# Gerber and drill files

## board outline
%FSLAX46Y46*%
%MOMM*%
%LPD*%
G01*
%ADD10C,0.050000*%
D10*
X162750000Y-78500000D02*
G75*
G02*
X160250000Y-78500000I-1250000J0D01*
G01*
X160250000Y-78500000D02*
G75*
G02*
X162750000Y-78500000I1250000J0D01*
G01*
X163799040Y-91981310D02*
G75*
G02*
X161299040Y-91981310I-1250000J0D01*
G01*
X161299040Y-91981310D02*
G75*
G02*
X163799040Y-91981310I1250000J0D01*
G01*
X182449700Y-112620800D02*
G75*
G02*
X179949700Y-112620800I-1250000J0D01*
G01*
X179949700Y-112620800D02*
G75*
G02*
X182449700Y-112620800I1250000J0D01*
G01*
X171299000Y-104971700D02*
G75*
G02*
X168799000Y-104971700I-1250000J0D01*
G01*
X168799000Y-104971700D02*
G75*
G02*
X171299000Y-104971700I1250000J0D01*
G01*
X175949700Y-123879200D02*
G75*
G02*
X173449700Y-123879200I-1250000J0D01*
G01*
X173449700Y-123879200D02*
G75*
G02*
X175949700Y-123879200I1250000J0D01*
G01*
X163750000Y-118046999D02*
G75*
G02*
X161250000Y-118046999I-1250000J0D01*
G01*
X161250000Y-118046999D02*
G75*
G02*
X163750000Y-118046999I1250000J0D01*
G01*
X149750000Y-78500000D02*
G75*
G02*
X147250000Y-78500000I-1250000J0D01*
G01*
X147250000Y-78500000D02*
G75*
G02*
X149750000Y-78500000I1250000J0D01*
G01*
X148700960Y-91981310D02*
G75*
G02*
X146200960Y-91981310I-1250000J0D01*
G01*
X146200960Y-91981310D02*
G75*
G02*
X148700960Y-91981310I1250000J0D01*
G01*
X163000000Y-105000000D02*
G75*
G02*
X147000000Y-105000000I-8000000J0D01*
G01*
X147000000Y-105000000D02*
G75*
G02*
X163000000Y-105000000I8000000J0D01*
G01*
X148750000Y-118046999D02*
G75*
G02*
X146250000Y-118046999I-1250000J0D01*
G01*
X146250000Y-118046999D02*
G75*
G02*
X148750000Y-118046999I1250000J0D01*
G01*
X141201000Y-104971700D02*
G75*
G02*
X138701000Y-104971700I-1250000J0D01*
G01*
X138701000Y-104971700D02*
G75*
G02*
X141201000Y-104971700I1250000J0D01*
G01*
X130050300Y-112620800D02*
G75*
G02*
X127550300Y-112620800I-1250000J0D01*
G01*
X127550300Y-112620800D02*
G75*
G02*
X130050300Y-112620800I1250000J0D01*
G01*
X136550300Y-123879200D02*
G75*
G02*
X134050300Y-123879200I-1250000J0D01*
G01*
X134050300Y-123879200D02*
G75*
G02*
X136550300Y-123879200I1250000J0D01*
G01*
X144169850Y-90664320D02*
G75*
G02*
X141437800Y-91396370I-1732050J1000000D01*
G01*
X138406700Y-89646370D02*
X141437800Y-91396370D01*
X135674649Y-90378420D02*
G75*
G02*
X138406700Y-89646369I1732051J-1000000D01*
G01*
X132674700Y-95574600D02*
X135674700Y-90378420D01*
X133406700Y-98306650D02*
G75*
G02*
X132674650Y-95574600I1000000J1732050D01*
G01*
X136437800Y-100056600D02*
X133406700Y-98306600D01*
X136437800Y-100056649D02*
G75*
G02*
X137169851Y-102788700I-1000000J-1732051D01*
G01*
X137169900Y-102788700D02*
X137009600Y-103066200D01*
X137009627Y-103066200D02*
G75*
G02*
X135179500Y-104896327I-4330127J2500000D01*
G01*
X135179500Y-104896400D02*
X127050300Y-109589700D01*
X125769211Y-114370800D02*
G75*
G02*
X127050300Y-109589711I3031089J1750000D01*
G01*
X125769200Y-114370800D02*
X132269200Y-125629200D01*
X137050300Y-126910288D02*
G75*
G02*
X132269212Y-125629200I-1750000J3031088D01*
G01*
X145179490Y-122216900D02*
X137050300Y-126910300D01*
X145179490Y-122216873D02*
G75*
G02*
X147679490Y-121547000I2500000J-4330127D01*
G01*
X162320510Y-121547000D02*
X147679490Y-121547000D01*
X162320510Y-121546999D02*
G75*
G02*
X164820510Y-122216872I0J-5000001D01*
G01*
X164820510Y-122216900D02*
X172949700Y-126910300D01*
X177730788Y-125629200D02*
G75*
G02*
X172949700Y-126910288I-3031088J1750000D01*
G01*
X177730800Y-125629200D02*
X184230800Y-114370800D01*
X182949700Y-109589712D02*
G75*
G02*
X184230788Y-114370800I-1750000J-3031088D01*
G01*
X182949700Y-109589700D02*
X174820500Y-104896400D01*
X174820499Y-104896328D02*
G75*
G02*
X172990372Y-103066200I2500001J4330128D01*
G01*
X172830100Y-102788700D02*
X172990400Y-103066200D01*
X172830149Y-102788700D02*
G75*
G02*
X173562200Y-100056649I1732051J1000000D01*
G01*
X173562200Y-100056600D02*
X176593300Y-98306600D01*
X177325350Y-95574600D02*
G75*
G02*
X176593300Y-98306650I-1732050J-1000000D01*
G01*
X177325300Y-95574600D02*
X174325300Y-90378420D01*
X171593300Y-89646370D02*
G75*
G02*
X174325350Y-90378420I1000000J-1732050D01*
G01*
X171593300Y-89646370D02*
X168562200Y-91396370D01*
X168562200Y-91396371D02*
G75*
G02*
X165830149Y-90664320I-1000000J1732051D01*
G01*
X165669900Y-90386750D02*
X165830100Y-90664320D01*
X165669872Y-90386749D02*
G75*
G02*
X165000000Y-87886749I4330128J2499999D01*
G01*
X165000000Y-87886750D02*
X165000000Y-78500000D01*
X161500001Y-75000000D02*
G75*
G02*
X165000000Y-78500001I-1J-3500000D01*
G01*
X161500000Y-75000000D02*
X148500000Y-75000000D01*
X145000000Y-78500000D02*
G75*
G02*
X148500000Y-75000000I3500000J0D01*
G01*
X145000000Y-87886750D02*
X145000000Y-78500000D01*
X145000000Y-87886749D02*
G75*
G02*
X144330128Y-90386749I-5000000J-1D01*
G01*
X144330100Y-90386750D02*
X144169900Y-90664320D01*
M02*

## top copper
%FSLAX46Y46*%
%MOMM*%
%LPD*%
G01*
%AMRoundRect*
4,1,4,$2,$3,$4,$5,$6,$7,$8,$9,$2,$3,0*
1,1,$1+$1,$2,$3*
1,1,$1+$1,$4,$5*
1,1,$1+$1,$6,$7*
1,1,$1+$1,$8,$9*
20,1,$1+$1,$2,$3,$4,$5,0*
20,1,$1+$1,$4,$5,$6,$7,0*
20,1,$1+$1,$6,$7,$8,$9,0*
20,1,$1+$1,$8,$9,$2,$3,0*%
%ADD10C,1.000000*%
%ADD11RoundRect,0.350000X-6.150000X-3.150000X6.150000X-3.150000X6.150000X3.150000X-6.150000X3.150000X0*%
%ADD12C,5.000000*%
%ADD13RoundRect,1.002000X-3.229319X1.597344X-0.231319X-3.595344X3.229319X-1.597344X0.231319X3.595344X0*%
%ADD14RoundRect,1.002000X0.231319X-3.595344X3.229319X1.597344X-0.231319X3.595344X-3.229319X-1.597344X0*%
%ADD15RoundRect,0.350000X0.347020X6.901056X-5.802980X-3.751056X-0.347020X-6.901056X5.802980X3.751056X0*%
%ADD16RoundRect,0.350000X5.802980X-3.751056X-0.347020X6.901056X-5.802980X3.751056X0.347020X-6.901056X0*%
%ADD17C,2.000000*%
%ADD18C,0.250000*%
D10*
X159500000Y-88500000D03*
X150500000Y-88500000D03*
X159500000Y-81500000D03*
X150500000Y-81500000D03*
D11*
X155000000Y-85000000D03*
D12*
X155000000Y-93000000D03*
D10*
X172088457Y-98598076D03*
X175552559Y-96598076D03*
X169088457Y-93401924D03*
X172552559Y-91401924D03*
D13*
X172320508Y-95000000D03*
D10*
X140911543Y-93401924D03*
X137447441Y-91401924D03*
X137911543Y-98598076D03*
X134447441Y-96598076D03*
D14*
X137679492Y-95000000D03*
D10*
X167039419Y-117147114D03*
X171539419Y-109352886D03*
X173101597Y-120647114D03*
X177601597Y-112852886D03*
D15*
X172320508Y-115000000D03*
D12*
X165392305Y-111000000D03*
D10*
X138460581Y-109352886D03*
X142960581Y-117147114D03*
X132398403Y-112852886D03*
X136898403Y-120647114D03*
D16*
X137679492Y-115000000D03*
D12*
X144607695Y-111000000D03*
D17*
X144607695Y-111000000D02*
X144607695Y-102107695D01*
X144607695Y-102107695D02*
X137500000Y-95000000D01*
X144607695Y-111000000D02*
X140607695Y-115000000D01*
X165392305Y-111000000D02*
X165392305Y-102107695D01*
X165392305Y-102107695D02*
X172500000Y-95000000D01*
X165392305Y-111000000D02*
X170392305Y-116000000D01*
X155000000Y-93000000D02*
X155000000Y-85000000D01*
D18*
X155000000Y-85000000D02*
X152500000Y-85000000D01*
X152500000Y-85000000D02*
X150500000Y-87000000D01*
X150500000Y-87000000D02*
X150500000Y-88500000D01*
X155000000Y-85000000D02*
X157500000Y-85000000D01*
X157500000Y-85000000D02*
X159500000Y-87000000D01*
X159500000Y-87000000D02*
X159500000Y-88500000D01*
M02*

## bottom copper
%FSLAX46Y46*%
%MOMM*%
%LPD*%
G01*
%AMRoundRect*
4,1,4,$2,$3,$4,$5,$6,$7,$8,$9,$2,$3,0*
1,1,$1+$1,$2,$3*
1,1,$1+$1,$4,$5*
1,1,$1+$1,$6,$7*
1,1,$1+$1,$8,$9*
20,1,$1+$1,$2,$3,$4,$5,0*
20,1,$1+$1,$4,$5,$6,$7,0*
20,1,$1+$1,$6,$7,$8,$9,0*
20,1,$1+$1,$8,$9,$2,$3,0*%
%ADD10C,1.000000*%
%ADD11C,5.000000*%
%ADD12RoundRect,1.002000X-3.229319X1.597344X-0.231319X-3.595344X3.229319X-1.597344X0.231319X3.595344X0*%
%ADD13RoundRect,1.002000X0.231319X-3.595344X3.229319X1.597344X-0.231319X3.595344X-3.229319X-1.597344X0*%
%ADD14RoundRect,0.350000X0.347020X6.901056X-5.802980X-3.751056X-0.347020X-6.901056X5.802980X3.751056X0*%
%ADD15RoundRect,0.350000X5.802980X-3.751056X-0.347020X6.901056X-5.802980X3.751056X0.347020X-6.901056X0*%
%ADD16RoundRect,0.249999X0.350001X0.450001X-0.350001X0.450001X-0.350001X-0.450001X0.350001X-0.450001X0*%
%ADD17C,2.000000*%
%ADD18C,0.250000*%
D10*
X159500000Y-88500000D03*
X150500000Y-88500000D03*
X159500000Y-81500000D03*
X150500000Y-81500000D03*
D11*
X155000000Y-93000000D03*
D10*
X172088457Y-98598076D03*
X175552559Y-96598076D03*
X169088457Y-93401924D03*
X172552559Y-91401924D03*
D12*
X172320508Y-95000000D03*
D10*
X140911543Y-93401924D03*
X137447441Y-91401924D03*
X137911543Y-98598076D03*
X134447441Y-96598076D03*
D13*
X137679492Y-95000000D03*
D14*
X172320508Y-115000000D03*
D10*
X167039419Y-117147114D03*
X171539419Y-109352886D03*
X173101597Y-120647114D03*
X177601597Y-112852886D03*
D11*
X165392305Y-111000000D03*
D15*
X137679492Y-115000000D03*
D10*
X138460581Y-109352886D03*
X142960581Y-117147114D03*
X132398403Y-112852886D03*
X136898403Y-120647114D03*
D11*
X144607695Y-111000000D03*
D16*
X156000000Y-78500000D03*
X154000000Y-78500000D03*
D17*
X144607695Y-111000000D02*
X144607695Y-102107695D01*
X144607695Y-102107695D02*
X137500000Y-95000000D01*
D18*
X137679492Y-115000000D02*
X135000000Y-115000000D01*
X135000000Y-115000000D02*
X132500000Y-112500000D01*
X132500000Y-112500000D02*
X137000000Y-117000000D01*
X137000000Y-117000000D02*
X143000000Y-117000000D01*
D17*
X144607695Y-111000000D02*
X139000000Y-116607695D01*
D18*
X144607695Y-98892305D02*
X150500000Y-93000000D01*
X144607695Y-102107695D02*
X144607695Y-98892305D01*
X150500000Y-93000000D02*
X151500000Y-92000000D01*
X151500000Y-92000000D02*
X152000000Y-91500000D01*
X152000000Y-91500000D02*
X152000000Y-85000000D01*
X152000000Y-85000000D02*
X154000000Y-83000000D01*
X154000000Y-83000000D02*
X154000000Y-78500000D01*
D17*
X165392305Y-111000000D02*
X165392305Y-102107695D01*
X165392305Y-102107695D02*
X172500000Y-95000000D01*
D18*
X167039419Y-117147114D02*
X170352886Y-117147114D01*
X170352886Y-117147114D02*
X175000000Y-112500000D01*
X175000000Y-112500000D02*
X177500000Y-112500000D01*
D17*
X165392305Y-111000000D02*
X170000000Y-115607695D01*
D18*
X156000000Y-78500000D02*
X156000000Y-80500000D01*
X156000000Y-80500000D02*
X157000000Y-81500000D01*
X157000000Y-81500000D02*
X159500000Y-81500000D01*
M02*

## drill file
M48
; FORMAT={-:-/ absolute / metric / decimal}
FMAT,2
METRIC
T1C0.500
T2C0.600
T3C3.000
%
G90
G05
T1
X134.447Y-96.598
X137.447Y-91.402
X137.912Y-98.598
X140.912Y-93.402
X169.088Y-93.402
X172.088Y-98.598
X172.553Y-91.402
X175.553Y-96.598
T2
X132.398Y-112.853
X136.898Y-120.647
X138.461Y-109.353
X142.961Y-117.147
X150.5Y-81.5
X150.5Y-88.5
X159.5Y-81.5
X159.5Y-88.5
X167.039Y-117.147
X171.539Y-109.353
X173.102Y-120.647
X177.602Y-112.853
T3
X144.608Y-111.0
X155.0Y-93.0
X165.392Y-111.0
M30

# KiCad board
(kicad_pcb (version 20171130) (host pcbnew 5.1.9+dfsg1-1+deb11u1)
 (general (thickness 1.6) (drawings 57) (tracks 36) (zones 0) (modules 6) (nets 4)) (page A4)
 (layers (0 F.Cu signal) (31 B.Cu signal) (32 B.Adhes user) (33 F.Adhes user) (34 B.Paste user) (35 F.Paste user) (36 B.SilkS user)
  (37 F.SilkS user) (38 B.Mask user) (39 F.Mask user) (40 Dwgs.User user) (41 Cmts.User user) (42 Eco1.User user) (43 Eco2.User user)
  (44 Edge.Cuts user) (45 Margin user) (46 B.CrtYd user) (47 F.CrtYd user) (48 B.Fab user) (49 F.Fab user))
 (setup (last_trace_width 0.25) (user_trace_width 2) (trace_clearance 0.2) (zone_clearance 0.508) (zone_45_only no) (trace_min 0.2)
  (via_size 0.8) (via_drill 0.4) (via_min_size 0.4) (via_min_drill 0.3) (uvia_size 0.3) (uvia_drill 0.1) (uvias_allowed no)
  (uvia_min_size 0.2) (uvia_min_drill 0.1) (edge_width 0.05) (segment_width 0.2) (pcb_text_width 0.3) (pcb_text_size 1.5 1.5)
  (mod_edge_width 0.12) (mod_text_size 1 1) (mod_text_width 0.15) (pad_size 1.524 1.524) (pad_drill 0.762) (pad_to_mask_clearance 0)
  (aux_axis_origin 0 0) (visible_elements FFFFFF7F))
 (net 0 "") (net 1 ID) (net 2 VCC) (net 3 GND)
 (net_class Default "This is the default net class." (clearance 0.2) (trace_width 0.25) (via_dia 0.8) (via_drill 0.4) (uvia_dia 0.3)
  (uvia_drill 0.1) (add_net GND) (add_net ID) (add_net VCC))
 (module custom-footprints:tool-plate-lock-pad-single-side (layer F.Cu) (at 155 105)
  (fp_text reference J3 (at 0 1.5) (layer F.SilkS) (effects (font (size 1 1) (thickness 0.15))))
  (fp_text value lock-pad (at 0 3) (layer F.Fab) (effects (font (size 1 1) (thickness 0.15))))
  (pad 1 thru_hole circle (at 4.5 -16.5) (size 1 1) (drill 0.6) (layers *.Cu *.Mask) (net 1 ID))
  (pad 1 thru_hole circle (at -4.5 -16.5) (size 1 1) (drill 0.6) (layers *.Cu *.Mask) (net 1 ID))
  (pad 1 thru_hole circle (at 4.5 -23.5) (size 1 1) (drill 0.6) (layers *.Cu *.Mask) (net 1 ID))
  (pad 1 thru_hole circle (at -4.5 -23.5) (size 1 1) (drill 0.6) (layers *.Cu *.Mask) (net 1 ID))
  (pad 1 smd roundrect (at 0 -20) (size 13 7) (layers F.Cu F.Paste F.Mask) (roundrect_rratio 0.05) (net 1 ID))
  (pad 1 thru_hole circle (at 0 -12) (size 5 5) (drill 3) (layers *.Cu *.Mask) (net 1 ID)))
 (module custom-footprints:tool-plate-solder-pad (layer F.Cu) (at 155 105 300)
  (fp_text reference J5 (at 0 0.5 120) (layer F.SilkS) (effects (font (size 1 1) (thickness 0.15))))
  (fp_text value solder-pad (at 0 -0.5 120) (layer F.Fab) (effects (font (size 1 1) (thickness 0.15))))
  (pad 1 thru_hole circle (at 3 -18 300) (size 1 1) (drill 0.5) (layers *.Cu *.Mask) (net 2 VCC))
  (pad 1 thru_hole circle (at 3 -22 300) (size 1 1) (drill 0.5) (layers *.Cu *.Mask) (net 2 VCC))
  (pad 1 thru_hole circle (at -3 -18 300) (size 1 1) (drill 0.5) (layers *.Cu *.Mask) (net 2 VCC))
  (pad 1 thru_hole circle (at -3 -22 300) (size 1 1) (drill 0.5) (layers *.Cu *.Mask) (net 2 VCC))
  (pad 1 smd roundrect (at 0 -20 300) (size 8 6) (layers B.Cu B.Paste B.Mask) (roundrect_rratio 0.167) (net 2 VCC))
  (pad 1 smd roundrect (at 0 -20 300) (size 8 6) (layers F.Cu F.Paste F.Mask) (roundrect_rratio 0.167) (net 2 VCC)))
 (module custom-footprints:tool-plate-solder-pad (layer F.Cu) (at 155 105 60)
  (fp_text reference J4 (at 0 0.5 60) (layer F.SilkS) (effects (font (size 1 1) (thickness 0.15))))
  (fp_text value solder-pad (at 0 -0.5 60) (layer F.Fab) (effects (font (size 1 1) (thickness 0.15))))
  (pad 1 thru_hole circle (at 3 -18 60) (size 1 1) (drill 0.5) (layers *.Cu *.Mask) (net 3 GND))
  (pad 1 thru_hole circle (at 3 -22 60) (size 1 1) (drill 0.5) (layers *.Cu *.Mask) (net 3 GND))
  (pad 1 thru_hole circle (at -3 -18 60) (size 1 1) (drill 0.5) (layers *.Cu *.Mask) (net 3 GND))
  (pad 1 thru_hole circle (at -3 -22 60) (size 1 1) (drill 0.5) (layers *.Cu *.Mask) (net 3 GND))
  (pad 1 smd roundrect (at 0 -20 60) (size 8 6) (layers B.Cu B.Paste B.Mask) (roundrect_rratio 0.167) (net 3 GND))
  (pad 1 smd roundrect (at 0 -20 60) (size 8 6) (layers F.Cu F.Paste F.Mask) (roundrect_rratio 0.167) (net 3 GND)))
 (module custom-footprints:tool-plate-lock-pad (layer F.Cu) (at 155 105 240)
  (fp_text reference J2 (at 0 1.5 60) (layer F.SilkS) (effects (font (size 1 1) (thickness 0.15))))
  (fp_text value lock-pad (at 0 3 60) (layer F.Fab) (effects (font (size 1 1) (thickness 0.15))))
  (pad 1 smd roundrect (at 0 -20 240) (size 13 7) (layers B.Cu B.Paste B.Mask) (roundrect_rratio 0.05) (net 2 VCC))
  (pad 1 thru_hole circle (at 4.5 -16.5 240) (size 1 1) (drill 0.6) (layers *.Cu *.Mask) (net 2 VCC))
  (pad 1 thru_hole circle (at -4.5 -16.5 240) (size 1 1) (drill 0.6) (layers *.Cu *.Mask) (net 2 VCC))
  (pad 1 thru_hole circle (at 4.5 -23.5 240) (size 1 1) (drill 0.6) (layers *.Cu *.Mask) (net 2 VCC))
  (pad 1 thru_hole circle (at -4.5 -23.5 240) (size 1 1) (drill 0.6) (layers *.Cu *.Mask) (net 2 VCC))
  (pad 1 smd roundrect (at 0 -20 240) (size 13 7) (layers F.Cu F.Paste F.Mask) (roundrect_rratio 0.05) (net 2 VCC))
  (pad 1 thru_hole circle (at 0 -12 240) (size 5 5) (drill 3) (layers *.Cu *.Mask) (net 2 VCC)))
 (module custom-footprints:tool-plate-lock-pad (layer F.Cu) (at 155 105 120)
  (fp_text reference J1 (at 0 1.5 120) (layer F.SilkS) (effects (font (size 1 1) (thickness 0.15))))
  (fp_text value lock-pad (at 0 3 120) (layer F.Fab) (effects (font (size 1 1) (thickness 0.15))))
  (pad 1 smd roundrect (at 0 -20 120) (size 13 7) (layers B.Cu B.Paste B.Mask) (roundrect_rratio 0.05) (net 3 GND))
  (pad 1 thru_hole circle (at 4.5 -16.5 120) (size 1 1) (drill 0.6) (layers *.Cu *.Mask) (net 3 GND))
  (pad 1 thru_hole circle (at -4.5 -16.5 120) (size 1 1) (drill 0.6) (layers *.Cu *.Mask) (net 3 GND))
  (pad 1 thru_hole circle (at 4.5 -23.5 120) (size 1 1) (drill 0.6) (layers *.Cu *.Mask) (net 3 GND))
  (pad 1 thru_hole circle (at -4.5 -23.5 120) (size 1 1) (drill 0.6) (layers *.Cu *.Mask) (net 3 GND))
  (pad 1 smd roundrect (at 0 -20 120) (size 13 7) (layers F.Cu F.Paste F.Mask) (roundrect_rratio 0.05) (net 3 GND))
  (pad 1 thru_hole circle (at 0 -12 120) (size 5 5) (drill 3) (layers *.Cu *.Mask) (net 3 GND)))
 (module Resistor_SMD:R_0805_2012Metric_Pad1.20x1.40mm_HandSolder (layer B.Cu) (at 155 78.5 180)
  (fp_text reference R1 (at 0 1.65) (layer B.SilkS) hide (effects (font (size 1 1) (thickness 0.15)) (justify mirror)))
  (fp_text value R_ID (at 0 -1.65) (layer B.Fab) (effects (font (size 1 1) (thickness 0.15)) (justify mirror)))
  (pad 1 smd roundrect (at -1 0 180) (size 1.2 1.4) (layers B.Cu B.Paste B.Mask) (roundrect_rratio 0.2083325) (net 1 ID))
  (pad 2 smd roundrect (at 1 0 180) (size 1.2 1.4) (layers B.Cu B.Paste B.Mask) (roundrect_rratio 0.2083325) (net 3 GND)))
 (gr_circle (center 161.5 78.5) (end 162.75 78.5) (layer Edge.Cuts) (width 0.05))
 (gr_circle (center 162.54904 91.98131) (end 163.79904 91.98131) (layer Edge.Cuts) (width 0.05))
 (gr_circle (center 181.1997 112.6208) (end 182.4497 112.6208) (layer Edge.Cuts) (width 0.05))
 (gr_circle (center 170.049 104.9717) (end 171.299 104.9717) (layer Edge.Cuts) (width 0.05))
 (gr_circle (center 174.6997 123.8792) (end 175.9497 123.8792) (layer Edge.Cuts) (width 0.05))
 (gr_circle (center 162.5 118.046999) (end 163.75 118.046999) (layer Edge.Cuts) (width 0.05))
 (gr_circle (center 148.5 78.5) (end 149.75 78.5) (layer Edge.Cuts) (width 0.05))
 (gr_circle (center 147.45096 91.98131) (end 148.70096 91.98131) (layer Edge.Cuts) (width 0.05))
 (gr_circle (center 155 105) (end 163 105) (layer Edge.Cuts) (width 0.05))
 (gr_circle (center 147.5 118.046999) (end 148.75 118.046999) (layer Edge.Cuts) (width 0.05))
 (gr_circle (center 139.951 104.9717) (end 141.201 104.9717) (layer Edge.Cuts) (width 0.05))
 (gr_circle (center 128.8003 112.6208) (end 130.0503 112.6208) (layer Edge.Cuts) (width 0.05))
 (gr_circle (center 135.3003 123.8792) (end 136.5503 123.8792) (layer Edge.Cuts) (width 0.05))
 (gr_arc (start 142.4378 89.66432) (end 141.4378 91.39637) (angle -90) (layer Edge.Cuts) (width 0.05))
 (gr_line (start 138.4067 89.64637) (end 141.4378 91.39637) (layer Edge.Cuts) (width 0.05))
 (gr_arc (start 137.4067 91.37842) (end 138.4067 89.646369) (angle -90) (layer Edge.Cuts) (width 0.05))
 (gr_line (start 132.6747 95.5746) (end 135.6747 90.37842) (layer Edge.Cuts) (width 0.05))
 (gr_arc (start 134.4067 96.5746) (end 132.67465 95.5746) (angle -90) (layer Edge.Cuts) (width 0.05))
 (gr_line (start 136.4378 100.0566) (end 133.4067 98.3066) (layer Edge.Cuts) (width 0.05))
 (gr_arc (start 135.4378 101.7887) (end 137.169851 102.7887) (angle -90) (layer Edge.Cuts) (width 0.05))
 (gr_line (start 137.1699 102.7887) (end 137.0096 103.0662) (layer Edge.Cuts) (width 0.05))
 (gr_arc (start 132.6795 100.5662) (end 135.1795 104.896327) (angle -30) (layer Edge.Cuts) (width 0.05))
 (gr_line (start 135.1795 104.8964) (end 127.0503 109.5897) (layer Edge.Cuts) (width 0.05))
 (gr_arc (start 128.8003 112.6208) (end 127.0503 109.589711) (angle -90) (layer Edge.Cuts) (width 0.05))
 (gr_line (start 125.7692 114.3708) (end 132.2692 125.6292) (layer Edge.Cuts) (width 0.05))
 (gr_arc (start 135.3003 123.8792) (end 132.269212 125.6292) (angle -90) (layer Edge.Cuts) (width 0.05))
 (gr_line (start 145.17949 122.2169) (end 137.0503 126.9103) (layer Edge.Cuts) (width 0.05))
 (gr_arc (start 147.67949 126.547) (end 147.67949 121.547) (angle -30) (layer Edge.Cuts) (width 0.05))
 (gr_line (start 162.32051 121.547) (end 147.67949 121.547) (layer Edge.Cuts) (width 0.05))
 (gr_arc (start 162.32051 126.547) (end 164.82051 122.216872) (angle -30) (layer Edge.Cuts) (width 0.05))
 (gr_line (start 164.82051 122.2169) (end 172.9497 126.9103) (layer Edge.Cuts) (width 0.05))
 (gr_arc (start 174.6997 123.8792) (end 172.9497 126.910288) (angle -90) (layer Edge.Cuts) (width 0.05))
 (gr_line (start 177.7308 125.6292) (end 184.2308 114.3708) (layer Edge.Cuts) (width 0.05))
 (gr_arc (start 181.1997 112.6208) (end 184.230788 114.3708) (angle -90) (layer Edge.Cuts) (width 0.05))
 (gr_line (start 182.9497 109.5897) (end 174.8205 104.8964) (layer Edge.Cuts) (width 0.05))
 (gr_arc (start 177.3205 100.5662) (end 172.990372 103.0662) (angle -30) (layer Edge.Cuts) (width 0.05))
 (gr_line (start 172.8301 102.7887) (end 172.9904 103.0662) (layer Edge.Cuts) (width 0.05))
 (gr_arc (start 174.5622 101.7887) (end 173.5622 100.056649) (angle -90) (layer Edge.Cuts) (width 0.05))
 (gr_line (start 173.5622 100.0566) (end 176.5933 98.3066) (layer Edge.Cuts) (width 0.05))
 (gr_arc (start 175.5933 96.5746) (end 176.5933 98.30665) (angle -90) (layer Edge.Cuts) (width 0.05))
 (gr_line (start 177.3253 95.5746) (end 174.3253 90.37842) (layer Edge.Cuts) (width 0.05))
 (gr_arc (start 172.5933 91.37842) (end 174.32535 90.37842) (angle -90) (layer Edge.Cuts) (width 0.05))
 (gr_line (start 171.5933 89.64637) (end 168.5622 91.39637) (layer Edge.Cuts) (width 0.05))
 (gr_arc (start 167.5622 89.66432) (end 165.830149 90.66432) (angle -90) (layer Edge.Cuts) (width 0.05))
 (gr_line (start 165.6699 90.38675) (end 165.8301 90.66432) (layer Edge.Cuts) (width 0.05))
 (gr_arc (start 170 87.88675) (end 165 87.886749) (angle -30) (layer Edge.Cuts) (width 0.05))
 (gr_line (start 165 87.88675) (end 165 78.5) (layer Edge.Cuts) (width 0.05))
 (gr_arc (start 161.5 78.5) (end 165 78.500001) (angle -90) (layer Edge.Cuts) (width 0.05))
 (gr_line (start 161.5 75) (end 148.5 75) (layer Edge.Cuts) (width 0.05))
 (gr_arc (start 148.5 78.5) (end 148.5 75) (angle -90) (layer Edge.Cuts) (width 0.05))
 (gr_line (start 145 87.88675) (end 145 78.5) (layer Edge.Cuts) (width 0.05))
 (gr_arc (start 140 87.88675) (end 144.330128 90.386749) (angle -30) (layer Edge.Cuts) (width 0.05))
 (gr_line (start 144.3301 90.38675) (end 144.1699 90.66432) (layer Edge.Cuts) (width 0.05))
 (segment (start 144.607695 111) (end 144.607695 102.107695) (width 2) (layer F.Cu) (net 3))
 (segment (start 144.607695 102.107695) (end 137.5 95) (width 2) (layer F.Cu) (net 3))
 (segment (start 144.607695 111) (end 144.607695 102.107695) (width 2) (layer B.Cu) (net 3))
 (segment (start 144.607695 102.107695) (end 137.5 95) (width 2) (layer B.Cu) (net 3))
 (segment (start 137.679492 115) (end 135 115) (width 0.25) (layer B.Cu) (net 3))
 (segment (start 135 115) (end 132.5 112.5) (width 0.25) (layer B.Cu) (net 3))
 (segment (start 132.5 112.5) (end 137 117) (width 0.25) (layer B.Cu) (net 3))
 (segment (start 137 117) (end 143 117) (width 0.25) (layer B.Cu) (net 3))
 (segment (start 144.607695 111) (end 140.607695 115) (width 2) (layer F.Cu) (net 3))
 (segment (start 144.607695 111) (end 139 116.607695) (width 2) (layer B.Cu) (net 3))
 (segment (start 144.607695 98.892305) (end 150.5 93) (width 0.25) (layer B.Cu) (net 3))
 (segment (start 144.607695 102.107695) (end 144.607695 98.892305) (width 0.25) (layer B.Cu) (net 3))
 (segment (start 150.5 93) (end 151.5 92) (width 0.25) (layer B.Cu) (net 3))
 (segment (start 151.5 92) (end 152 91.5) (width 0.25) (layer B.Cu) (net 3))
 (segment (start 152 91.5) (end 152 85) (width 0.25) (layer B.Cu) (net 3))
 (segment (start 152 85) (end 154 83) (width 0.25) (layer B.Cu) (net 3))
 (segment (start 154 83) (end 154 78.5) (width 0.25) (layer B.Cu) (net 3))
 (segment (start 165.392305 111) (end 165.392305 102.107695) (width 2) (layer F.Cu) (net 2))
 (segment (start 165.392305 102.107695) (end 172.5 95) (width 2) (layer F.Cu) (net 2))
 (segment (start 165.392305 111) (end 165.392305 102.107695) (width 2) (layer B.Cu) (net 2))
 (segment (start 165.392305 102.107695) (end 172.5 95) (width 2) (layer B.Cu) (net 2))
 (segment (start 167.039419 117.147114) (end 170.352886 117.147114) (width 0.25) (layer B.Cu) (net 2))
 (segment (start 170.352886 117.147114) (end 175 112.5) (width 0.25) (layer B.Cu) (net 2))
 (segment (start 175 112.5) (end 177.5 112.5) (width 0.25) (layer B.Cu) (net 2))
 (segment (start 165.392305 111) (end 170.392305 116) (width 2) (layer F.Cu) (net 2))
 (segment (start 165.392305 111) (end 170 115.607695) (width 2) (layer B.Cu) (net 2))
 (segment (start 155 93) (end 155 85) (width 2) (layer F.Cu) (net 1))
 (segment (start 156 78.5) (end 156 80.5) (width 0.25) (layer B.Cu) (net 1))
 (segment (start 156 80.5) (end 157 81.5) (width 0.25) (layer B.Cu) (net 1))
 (segment (start 157 81.5) (end 159.5 81.5) (width 0.25) (layer B.Cu) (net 1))
 (segment (start 155 85) (end 152.5 85) (width 0.25) (layer F.Cu) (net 1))
 (segment (start 152.5 85) (end 150.5 87) (width 0.25) (layer F.Cu) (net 1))
 (segment (start 150.5 87) (end 150.5 88.5) (width 0.25) (layer F.Cu) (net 1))
 (segment (start 155 85) (end 157.5 85) (width 0.25) (layer F.Cu) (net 1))
 (segment (start 157.5 85) (end 159.5 87) (width 0.25) (layer F.Cu) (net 1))
 (segment (start 159.5 87) (end 159.5 88.5) (width 0.25) (layer F.Cu) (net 1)))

